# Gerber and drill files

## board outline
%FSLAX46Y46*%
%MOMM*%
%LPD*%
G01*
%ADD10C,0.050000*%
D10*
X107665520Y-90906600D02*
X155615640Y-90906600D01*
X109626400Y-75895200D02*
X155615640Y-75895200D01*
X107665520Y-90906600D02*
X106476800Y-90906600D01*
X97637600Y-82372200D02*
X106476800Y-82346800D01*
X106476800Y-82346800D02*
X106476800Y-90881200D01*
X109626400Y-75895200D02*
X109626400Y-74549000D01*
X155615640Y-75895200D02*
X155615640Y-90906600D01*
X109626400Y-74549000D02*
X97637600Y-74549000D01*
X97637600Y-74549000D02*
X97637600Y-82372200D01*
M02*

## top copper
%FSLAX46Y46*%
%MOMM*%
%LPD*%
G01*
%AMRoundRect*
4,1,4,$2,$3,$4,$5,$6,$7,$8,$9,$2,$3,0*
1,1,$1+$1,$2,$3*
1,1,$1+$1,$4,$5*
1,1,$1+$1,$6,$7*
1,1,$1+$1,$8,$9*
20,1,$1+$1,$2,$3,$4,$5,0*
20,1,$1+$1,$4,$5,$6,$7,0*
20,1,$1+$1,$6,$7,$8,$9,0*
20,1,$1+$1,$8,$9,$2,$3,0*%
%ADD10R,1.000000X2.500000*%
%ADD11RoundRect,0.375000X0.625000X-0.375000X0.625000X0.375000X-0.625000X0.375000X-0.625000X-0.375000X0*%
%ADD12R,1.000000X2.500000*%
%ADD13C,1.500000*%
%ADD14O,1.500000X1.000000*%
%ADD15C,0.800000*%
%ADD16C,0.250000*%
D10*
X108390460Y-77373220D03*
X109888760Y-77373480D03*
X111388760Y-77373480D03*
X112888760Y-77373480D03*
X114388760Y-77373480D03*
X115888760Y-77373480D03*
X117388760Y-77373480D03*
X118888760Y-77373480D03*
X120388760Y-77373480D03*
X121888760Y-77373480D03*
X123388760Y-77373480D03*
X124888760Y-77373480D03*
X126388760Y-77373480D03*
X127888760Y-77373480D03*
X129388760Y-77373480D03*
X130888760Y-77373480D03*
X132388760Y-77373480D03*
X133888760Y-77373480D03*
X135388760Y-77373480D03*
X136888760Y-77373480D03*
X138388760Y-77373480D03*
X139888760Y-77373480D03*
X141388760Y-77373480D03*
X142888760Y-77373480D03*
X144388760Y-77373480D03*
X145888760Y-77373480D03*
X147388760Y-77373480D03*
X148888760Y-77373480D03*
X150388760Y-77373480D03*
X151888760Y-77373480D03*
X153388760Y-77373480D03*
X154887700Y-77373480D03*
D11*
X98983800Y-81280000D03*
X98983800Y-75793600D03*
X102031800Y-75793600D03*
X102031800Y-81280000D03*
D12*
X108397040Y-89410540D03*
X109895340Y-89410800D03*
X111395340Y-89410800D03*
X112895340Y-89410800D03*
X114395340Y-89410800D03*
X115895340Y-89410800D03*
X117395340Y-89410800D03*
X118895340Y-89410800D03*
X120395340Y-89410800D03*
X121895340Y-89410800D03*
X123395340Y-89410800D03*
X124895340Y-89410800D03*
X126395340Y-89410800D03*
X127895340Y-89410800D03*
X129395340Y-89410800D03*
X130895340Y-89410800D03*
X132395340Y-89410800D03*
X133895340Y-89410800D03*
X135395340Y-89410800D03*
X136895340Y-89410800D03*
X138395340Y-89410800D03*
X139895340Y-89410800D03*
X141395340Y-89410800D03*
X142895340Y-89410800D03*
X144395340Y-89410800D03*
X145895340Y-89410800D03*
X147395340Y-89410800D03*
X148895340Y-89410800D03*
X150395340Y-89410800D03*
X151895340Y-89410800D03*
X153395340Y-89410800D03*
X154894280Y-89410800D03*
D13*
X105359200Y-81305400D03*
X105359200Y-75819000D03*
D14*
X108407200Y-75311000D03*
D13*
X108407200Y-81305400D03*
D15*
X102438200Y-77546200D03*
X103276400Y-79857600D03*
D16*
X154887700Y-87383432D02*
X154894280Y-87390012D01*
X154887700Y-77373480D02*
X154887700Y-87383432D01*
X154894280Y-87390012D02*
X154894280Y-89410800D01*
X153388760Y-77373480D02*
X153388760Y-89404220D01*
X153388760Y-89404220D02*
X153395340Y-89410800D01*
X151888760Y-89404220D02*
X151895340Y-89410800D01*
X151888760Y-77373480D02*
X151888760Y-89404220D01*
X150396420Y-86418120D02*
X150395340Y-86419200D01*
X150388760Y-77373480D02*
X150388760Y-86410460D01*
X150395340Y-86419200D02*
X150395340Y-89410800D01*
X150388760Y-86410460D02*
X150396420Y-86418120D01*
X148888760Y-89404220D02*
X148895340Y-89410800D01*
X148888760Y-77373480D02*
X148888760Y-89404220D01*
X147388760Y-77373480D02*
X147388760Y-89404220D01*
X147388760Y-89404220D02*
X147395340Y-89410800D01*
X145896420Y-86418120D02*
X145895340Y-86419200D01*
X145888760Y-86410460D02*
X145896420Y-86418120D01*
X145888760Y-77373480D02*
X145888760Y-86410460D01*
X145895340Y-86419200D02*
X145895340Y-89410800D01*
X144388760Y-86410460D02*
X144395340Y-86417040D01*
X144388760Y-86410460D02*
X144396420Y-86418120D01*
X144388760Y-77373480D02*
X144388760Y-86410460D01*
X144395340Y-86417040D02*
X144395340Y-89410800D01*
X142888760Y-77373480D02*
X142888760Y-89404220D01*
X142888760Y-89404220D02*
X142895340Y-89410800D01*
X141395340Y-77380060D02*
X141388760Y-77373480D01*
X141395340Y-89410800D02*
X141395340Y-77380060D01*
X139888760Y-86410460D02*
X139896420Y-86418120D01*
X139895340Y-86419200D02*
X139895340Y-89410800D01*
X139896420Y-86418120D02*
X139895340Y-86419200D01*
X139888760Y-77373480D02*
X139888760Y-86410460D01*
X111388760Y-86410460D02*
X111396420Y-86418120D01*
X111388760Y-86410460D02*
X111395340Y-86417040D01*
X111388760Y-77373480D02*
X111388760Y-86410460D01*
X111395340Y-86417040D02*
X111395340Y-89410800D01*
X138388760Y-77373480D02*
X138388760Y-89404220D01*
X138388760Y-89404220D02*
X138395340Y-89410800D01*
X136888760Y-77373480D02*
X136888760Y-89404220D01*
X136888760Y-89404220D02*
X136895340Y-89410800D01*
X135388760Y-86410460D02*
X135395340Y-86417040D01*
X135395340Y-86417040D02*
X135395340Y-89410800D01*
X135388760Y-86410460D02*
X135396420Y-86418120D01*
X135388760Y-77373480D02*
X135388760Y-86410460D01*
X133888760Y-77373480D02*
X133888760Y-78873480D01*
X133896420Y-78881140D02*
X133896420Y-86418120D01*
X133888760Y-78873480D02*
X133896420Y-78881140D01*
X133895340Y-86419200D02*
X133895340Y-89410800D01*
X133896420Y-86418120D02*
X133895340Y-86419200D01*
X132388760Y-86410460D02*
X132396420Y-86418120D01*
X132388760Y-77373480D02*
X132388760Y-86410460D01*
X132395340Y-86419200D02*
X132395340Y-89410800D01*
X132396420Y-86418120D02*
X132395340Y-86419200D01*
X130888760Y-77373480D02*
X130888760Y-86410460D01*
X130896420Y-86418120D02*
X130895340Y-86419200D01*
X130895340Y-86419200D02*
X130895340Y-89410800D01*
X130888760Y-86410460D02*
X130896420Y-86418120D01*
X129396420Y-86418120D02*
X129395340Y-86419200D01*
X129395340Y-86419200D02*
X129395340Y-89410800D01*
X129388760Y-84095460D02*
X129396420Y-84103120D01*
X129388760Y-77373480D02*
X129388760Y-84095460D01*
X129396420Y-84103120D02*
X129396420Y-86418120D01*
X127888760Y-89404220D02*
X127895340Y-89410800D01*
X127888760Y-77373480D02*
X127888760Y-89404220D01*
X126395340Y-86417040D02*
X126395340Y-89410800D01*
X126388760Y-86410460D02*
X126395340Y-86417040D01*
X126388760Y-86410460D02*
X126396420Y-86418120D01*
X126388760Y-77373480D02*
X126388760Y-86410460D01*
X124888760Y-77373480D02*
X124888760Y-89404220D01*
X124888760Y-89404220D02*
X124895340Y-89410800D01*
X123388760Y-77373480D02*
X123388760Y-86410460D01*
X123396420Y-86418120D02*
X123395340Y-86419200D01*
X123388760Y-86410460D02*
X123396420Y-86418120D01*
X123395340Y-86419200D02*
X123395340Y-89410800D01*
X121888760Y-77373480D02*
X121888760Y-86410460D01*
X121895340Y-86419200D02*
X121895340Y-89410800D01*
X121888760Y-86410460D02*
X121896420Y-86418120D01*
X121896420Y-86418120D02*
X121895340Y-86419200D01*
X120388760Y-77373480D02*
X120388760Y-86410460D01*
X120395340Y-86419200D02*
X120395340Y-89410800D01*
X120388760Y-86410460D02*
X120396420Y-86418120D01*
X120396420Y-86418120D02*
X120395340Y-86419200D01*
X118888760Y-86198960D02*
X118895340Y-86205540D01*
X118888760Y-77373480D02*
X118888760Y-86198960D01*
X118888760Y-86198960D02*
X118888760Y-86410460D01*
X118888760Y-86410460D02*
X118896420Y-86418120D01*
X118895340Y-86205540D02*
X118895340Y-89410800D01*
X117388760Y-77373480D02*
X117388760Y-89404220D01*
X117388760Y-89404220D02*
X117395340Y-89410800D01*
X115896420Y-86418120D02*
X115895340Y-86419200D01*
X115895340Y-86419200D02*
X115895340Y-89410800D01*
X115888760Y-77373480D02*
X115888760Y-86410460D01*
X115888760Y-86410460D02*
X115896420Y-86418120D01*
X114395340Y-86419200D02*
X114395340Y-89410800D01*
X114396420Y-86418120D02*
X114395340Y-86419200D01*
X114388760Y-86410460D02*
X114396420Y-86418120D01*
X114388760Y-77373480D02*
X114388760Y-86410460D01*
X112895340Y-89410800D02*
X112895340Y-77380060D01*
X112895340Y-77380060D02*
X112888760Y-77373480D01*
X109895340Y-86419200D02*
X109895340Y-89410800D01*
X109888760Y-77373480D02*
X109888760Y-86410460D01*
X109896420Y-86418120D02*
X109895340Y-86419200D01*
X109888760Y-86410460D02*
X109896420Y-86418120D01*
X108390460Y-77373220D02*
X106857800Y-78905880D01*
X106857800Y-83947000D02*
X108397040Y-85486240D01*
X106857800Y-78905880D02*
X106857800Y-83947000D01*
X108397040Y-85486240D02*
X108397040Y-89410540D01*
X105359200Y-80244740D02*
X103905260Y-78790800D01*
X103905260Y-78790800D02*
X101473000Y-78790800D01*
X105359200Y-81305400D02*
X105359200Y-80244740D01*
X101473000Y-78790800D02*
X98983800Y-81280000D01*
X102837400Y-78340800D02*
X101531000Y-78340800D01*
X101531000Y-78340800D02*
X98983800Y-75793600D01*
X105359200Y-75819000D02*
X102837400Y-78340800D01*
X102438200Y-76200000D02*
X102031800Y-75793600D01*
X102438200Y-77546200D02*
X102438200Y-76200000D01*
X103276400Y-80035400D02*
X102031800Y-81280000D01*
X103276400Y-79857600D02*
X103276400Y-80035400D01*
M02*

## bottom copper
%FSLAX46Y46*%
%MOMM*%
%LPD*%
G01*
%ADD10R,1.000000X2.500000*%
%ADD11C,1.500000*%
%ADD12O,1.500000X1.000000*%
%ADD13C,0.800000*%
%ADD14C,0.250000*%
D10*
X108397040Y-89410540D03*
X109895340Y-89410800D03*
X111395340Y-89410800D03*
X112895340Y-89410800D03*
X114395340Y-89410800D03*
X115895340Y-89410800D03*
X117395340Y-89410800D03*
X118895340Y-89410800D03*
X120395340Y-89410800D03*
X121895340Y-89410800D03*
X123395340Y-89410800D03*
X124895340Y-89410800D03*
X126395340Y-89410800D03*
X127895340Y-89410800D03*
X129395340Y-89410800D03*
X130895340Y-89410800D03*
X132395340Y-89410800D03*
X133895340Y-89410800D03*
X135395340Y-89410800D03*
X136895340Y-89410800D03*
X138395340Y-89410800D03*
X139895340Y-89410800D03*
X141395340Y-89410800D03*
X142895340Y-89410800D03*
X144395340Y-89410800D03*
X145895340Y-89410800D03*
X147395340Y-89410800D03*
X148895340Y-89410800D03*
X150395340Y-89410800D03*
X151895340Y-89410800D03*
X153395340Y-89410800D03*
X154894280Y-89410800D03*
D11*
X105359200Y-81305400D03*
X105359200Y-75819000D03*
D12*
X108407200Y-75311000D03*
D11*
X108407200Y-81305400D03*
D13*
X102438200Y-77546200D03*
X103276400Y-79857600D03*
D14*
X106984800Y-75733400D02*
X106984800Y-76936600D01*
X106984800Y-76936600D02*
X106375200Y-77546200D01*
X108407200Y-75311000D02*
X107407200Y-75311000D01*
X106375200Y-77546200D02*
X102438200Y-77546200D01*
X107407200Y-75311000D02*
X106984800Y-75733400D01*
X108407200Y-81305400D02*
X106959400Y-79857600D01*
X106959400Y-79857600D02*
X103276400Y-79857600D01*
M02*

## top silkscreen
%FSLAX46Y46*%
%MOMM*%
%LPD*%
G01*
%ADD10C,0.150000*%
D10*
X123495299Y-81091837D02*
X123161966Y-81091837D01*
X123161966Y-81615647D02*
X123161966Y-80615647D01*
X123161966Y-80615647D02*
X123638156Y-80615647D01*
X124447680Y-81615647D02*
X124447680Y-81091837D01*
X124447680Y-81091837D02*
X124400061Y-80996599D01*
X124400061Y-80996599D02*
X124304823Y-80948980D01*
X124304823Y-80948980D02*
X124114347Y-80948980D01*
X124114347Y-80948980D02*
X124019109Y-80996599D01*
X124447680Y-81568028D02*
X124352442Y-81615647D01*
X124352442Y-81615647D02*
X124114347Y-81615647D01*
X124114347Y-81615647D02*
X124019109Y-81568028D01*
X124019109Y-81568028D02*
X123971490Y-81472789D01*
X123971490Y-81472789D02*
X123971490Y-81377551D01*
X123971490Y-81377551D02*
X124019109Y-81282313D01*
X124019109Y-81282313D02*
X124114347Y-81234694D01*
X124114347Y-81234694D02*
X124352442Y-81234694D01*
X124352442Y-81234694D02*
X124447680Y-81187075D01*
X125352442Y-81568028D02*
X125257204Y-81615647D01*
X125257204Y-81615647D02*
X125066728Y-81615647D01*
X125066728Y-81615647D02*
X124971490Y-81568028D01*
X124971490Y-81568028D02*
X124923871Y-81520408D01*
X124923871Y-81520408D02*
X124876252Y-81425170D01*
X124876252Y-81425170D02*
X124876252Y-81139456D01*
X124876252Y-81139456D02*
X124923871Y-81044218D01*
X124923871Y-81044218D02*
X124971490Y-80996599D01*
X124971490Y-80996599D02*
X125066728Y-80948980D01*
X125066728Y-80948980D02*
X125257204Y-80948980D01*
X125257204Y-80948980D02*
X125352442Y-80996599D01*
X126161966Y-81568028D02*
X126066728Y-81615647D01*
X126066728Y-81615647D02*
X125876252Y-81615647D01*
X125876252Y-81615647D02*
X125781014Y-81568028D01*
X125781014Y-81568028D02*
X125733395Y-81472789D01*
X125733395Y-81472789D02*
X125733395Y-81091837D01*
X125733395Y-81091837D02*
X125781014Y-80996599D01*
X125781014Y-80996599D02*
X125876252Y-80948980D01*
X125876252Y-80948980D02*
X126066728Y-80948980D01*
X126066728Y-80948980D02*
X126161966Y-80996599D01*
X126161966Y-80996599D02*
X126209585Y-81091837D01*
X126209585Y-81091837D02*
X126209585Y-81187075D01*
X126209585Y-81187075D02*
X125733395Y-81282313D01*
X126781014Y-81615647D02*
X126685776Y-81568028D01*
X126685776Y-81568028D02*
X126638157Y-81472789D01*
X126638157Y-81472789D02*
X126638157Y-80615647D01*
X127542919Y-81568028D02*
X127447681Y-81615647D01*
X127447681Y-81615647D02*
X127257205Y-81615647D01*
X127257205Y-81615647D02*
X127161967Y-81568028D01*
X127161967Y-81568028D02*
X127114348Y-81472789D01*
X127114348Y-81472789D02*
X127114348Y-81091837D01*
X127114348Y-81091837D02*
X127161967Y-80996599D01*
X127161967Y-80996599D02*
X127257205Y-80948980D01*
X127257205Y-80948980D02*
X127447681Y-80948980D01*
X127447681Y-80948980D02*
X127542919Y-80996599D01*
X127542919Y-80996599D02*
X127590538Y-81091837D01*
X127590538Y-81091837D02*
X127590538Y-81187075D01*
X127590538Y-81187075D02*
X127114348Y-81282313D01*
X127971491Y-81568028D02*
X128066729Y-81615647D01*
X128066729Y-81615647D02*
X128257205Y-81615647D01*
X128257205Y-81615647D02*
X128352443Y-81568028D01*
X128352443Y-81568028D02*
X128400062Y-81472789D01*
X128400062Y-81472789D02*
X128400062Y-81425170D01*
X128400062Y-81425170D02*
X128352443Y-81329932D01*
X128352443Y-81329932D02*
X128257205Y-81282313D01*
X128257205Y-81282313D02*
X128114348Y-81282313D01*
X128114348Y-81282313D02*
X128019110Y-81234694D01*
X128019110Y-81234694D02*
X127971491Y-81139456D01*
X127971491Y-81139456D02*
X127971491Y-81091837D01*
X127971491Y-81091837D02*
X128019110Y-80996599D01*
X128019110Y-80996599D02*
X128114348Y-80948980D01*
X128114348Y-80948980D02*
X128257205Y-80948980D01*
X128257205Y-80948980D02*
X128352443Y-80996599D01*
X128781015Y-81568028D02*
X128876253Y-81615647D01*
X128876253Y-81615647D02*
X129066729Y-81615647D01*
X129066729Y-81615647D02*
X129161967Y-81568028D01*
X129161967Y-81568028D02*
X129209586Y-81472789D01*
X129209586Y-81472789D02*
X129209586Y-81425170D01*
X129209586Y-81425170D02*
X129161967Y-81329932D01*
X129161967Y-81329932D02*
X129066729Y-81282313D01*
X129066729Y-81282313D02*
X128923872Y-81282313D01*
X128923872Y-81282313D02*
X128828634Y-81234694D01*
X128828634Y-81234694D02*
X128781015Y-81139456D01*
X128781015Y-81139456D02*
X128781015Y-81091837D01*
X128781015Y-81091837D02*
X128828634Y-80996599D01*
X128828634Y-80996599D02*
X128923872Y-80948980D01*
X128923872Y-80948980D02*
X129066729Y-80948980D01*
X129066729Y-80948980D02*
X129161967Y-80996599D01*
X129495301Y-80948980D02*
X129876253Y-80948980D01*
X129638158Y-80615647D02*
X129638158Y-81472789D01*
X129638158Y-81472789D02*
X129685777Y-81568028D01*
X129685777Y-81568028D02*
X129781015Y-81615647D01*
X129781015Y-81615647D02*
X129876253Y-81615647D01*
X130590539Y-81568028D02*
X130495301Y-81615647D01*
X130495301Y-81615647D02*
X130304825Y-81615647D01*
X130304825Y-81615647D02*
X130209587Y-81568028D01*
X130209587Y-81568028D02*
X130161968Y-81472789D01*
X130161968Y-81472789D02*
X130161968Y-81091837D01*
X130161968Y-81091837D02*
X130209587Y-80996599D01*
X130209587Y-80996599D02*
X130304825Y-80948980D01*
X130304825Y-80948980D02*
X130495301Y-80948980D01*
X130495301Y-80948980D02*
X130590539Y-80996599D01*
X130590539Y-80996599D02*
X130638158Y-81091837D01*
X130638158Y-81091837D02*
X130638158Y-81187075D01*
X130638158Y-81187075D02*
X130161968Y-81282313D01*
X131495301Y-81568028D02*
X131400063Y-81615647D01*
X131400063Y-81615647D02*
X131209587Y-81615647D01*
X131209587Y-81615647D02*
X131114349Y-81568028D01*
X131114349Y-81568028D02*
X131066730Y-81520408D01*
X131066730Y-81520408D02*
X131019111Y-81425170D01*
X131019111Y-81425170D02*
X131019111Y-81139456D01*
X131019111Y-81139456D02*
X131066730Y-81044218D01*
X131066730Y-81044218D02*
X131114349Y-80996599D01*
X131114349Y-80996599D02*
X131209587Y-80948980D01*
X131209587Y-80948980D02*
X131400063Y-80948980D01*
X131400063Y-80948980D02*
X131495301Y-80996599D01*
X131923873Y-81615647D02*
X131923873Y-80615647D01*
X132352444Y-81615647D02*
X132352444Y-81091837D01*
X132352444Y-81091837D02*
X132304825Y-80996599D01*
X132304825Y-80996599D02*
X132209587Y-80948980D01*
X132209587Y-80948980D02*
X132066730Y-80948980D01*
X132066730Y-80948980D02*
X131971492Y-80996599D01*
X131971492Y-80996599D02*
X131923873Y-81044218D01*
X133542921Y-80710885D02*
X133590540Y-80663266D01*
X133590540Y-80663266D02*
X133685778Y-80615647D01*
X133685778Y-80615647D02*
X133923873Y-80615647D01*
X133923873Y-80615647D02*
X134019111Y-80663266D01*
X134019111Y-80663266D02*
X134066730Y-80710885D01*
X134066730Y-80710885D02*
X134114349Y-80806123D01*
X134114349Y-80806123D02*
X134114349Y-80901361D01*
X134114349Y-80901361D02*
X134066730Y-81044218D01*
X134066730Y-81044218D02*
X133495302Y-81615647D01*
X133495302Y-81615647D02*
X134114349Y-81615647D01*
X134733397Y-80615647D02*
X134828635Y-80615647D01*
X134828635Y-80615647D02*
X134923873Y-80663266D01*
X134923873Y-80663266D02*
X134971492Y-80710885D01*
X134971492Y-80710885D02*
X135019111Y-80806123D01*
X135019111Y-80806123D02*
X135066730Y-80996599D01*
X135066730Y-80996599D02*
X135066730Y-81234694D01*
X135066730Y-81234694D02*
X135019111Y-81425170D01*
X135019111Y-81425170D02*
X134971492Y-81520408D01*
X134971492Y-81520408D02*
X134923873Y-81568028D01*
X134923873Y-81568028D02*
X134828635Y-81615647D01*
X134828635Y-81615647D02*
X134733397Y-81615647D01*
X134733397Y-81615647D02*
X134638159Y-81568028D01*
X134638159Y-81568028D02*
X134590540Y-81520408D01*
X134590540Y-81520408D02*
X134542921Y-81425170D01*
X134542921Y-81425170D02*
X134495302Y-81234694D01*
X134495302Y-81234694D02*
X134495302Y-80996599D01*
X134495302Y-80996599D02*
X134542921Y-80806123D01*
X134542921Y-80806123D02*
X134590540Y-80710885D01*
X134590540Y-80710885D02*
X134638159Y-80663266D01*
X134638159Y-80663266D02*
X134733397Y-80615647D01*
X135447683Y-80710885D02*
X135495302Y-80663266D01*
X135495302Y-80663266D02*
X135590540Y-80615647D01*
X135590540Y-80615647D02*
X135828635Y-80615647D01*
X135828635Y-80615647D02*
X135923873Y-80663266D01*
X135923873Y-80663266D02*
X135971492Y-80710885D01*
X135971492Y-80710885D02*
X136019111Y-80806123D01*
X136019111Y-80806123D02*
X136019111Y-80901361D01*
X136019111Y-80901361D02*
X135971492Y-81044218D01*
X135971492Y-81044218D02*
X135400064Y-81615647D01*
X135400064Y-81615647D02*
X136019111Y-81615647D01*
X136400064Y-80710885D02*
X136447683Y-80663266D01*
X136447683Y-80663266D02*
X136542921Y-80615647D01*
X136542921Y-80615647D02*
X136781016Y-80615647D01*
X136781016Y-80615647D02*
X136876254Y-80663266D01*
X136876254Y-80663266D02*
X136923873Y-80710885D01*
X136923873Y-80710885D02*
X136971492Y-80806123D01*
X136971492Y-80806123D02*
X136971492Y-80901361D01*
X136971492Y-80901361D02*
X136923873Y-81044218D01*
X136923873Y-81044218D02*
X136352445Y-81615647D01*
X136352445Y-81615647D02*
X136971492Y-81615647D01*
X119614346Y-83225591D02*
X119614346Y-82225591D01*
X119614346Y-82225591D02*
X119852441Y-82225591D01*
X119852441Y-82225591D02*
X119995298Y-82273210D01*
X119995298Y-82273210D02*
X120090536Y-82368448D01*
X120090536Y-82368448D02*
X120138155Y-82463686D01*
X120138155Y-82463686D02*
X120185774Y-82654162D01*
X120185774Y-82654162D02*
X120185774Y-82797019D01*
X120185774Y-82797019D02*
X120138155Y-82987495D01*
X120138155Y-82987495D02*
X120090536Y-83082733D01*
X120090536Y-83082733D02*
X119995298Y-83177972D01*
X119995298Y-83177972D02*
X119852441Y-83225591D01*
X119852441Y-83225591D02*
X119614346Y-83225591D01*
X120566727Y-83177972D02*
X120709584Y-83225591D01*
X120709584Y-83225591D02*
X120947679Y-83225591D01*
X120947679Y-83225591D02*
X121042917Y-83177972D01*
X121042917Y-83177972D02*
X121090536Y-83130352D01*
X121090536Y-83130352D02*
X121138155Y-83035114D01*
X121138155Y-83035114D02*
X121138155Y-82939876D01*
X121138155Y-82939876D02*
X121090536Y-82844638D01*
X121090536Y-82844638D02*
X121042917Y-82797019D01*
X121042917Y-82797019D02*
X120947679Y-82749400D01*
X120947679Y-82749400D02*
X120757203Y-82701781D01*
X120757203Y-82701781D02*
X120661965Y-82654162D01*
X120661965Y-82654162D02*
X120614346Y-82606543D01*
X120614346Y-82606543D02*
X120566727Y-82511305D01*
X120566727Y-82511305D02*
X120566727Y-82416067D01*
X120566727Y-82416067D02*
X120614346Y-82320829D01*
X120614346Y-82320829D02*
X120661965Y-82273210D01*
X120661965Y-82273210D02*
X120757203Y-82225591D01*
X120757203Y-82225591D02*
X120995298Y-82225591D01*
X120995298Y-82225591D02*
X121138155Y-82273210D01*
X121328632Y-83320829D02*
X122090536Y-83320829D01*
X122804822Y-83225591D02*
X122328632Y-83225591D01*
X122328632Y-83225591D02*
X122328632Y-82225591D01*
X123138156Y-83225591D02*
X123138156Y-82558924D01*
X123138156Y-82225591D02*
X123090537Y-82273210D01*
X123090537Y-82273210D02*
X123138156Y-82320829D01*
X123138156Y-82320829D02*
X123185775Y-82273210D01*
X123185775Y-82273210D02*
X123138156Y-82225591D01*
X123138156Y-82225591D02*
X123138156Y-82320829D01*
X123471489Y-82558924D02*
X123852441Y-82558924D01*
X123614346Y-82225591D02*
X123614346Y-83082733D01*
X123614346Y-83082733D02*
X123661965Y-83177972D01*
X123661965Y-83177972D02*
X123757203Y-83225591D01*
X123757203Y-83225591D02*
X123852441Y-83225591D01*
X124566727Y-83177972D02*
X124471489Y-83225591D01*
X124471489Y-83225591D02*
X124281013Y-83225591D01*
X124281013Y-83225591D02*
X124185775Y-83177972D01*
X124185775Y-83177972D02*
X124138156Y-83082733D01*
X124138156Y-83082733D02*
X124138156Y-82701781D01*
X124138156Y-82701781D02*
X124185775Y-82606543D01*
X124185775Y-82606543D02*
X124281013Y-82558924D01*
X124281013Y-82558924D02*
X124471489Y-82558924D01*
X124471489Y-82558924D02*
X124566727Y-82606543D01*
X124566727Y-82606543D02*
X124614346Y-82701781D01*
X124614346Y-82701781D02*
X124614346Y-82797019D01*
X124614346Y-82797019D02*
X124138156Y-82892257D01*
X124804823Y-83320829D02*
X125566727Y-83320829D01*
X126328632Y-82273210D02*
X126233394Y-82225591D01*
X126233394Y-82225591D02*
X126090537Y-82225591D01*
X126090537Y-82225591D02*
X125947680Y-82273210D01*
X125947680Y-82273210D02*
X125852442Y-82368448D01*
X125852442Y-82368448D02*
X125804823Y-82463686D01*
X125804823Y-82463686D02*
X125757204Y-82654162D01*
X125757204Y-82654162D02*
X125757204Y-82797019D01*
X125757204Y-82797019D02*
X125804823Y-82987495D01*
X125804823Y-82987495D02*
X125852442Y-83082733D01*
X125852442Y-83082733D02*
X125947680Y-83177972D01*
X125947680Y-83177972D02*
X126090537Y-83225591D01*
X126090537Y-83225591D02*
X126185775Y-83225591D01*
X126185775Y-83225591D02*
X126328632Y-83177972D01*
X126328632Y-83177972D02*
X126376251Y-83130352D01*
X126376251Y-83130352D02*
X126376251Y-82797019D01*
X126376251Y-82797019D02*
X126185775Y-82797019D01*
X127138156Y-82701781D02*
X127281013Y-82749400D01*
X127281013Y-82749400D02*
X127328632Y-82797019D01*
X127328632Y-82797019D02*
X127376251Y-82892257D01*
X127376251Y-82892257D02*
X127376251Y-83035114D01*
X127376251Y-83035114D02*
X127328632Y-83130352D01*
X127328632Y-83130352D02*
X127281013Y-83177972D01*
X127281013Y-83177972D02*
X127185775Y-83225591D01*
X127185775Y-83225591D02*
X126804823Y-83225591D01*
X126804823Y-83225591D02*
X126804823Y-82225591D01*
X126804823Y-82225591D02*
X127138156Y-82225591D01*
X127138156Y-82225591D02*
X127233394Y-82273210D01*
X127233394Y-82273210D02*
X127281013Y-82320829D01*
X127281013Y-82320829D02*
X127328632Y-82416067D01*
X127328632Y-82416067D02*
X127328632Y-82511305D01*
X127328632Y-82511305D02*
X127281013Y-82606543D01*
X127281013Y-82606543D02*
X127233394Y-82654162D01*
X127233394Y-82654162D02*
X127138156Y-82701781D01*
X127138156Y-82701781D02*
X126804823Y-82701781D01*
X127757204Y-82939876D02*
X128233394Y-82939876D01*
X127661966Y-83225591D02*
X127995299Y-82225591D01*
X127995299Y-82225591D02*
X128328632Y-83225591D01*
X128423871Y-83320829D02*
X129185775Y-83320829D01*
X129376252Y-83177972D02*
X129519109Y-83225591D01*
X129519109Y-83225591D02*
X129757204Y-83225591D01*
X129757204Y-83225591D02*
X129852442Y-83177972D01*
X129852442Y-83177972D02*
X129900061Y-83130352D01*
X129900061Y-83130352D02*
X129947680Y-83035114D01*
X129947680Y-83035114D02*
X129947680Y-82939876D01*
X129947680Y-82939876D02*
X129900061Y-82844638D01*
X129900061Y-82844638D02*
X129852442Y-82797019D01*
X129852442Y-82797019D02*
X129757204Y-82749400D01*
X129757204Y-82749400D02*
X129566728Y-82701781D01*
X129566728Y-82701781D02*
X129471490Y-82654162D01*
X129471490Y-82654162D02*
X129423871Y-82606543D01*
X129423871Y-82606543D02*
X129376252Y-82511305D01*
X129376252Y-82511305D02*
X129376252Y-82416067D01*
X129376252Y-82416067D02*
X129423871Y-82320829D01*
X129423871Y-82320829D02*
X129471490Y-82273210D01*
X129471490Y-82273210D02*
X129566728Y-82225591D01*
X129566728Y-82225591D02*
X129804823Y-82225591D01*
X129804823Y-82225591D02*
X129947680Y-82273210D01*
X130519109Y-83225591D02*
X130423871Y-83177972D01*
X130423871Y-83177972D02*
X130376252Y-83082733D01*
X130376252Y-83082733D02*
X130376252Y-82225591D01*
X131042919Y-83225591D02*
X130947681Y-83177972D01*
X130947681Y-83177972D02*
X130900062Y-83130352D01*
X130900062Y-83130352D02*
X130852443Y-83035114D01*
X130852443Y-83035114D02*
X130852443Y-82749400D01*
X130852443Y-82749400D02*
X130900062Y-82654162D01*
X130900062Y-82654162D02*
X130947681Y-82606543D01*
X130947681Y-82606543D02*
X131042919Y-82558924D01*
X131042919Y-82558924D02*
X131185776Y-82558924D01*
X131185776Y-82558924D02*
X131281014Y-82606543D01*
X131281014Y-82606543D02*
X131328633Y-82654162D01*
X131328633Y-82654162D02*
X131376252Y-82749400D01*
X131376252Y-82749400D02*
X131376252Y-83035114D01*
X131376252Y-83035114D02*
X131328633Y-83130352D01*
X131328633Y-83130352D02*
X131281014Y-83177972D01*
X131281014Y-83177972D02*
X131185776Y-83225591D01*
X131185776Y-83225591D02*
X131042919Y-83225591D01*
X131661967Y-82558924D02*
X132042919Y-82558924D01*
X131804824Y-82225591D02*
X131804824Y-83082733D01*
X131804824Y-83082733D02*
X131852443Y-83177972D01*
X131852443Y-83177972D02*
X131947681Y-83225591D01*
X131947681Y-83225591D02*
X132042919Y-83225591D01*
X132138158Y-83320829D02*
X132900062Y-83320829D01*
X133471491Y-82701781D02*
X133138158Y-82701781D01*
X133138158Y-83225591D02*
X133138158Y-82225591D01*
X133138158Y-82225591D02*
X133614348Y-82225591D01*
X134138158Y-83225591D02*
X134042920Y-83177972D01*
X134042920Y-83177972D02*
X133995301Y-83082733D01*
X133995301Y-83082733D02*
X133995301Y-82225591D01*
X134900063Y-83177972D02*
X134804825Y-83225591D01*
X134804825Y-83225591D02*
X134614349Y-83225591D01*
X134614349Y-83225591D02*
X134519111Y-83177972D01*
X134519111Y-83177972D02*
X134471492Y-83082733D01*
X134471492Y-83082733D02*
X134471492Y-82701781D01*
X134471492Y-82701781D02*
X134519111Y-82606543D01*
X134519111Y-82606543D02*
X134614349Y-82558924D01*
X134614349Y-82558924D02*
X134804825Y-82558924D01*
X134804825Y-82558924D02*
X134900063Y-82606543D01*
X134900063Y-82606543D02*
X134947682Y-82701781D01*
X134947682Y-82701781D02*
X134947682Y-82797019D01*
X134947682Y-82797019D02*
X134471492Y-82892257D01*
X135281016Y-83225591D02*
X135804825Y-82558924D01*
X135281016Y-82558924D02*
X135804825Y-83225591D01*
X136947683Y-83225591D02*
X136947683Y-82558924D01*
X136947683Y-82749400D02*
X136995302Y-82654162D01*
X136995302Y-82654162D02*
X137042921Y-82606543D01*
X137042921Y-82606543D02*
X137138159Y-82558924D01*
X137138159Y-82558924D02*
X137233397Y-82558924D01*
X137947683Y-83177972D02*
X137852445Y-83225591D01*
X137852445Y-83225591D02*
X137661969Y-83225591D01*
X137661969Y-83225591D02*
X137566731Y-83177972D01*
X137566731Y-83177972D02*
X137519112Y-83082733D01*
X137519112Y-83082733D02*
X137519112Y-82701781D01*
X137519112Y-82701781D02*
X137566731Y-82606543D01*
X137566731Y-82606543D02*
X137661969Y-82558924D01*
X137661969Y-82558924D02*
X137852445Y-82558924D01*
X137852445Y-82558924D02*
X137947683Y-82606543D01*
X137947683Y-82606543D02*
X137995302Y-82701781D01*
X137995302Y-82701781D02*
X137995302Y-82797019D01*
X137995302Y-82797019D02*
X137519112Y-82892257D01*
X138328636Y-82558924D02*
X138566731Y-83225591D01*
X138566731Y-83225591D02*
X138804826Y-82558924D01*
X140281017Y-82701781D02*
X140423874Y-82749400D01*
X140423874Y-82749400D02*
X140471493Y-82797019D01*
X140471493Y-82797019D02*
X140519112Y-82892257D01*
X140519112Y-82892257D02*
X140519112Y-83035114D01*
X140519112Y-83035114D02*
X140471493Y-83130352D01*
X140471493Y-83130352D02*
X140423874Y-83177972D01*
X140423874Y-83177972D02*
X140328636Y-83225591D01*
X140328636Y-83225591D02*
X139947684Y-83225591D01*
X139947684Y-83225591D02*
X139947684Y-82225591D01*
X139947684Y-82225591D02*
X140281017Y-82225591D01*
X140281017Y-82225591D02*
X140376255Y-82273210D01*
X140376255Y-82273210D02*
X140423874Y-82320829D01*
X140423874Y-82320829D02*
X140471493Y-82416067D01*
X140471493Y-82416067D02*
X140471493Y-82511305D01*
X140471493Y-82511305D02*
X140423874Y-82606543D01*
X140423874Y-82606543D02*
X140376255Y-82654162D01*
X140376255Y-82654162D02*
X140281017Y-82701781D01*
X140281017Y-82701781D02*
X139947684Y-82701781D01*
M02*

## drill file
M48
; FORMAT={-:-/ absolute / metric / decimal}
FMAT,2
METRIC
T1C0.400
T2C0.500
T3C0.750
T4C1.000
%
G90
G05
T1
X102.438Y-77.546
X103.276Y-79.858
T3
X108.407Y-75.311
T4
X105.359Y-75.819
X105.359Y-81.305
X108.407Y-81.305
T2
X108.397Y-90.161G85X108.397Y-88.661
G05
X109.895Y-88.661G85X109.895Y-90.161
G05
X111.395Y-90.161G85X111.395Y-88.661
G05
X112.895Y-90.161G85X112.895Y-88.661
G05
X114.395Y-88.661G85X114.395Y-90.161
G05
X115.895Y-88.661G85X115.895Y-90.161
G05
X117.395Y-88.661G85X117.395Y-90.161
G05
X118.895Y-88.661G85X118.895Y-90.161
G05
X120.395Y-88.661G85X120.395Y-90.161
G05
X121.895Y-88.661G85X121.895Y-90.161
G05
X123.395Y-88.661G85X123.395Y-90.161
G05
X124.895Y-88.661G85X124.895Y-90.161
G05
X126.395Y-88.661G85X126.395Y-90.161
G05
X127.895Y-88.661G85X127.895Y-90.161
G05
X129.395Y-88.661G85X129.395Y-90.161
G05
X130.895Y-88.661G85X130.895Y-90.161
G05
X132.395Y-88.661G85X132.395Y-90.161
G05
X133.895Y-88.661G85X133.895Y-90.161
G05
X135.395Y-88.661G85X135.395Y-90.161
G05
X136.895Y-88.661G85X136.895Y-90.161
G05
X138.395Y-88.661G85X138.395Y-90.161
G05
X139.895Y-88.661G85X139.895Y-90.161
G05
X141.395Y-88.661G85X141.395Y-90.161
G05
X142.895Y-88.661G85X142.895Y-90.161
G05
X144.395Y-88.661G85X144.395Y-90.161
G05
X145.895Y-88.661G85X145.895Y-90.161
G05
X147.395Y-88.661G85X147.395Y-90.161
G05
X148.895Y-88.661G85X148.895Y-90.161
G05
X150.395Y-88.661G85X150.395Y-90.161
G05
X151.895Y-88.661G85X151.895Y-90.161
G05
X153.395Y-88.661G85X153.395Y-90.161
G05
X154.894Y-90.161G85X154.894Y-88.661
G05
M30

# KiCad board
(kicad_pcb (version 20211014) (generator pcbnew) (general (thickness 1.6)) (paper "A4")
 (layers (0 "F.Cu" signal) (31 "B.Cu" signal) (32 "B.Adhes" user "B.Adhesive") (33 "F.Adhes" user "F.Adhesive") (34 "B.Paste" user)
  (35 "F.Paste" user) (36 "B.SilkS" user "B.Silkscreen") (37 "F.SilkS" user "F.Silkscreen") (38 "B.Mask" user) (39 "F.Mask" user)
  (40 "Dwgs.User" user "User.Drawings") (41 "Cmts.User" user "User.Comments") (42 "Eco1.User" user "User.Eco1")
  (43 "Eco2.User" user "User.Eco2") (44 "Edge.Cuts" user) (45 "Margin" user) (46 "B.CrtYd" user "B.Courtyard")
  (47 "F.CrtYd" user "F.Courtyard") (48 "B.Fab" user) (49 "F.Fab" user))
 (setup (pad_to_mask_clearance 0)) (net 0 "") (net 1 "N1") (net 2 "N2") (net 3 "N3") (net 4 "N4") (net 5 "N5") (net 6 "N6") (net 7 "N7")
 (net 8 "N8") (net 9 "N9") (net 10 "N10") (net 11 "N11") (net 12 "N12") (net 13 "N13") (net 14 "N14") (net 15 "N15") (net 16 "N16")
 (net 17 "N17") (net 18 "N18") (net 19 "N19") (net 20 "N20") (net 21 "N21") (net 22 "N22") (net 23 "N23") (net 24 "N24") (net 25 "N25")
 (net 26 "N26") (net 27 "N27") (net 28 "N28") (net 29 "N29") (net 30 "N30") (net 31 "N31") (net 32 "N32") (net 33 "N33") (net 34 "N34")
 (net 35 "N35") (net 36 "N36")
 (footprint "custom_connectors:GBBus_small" (layer "F.Cu") (at 130.11762 77.37068)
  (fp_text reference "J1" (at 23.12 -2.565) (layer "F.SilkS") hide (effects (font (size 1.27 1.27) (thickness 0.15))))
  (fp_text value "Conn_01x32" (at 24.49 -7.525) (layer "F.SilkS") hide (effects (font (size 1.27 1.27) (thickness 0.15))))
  (pad "1" smd rect locked (at -21.72716 0.00254 180) (size 1 2.5) (layers "F.Cu" "F.Paste" "F.Mask") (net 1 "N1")
   (solder_mask_margin 0.0508))
  (pad "2" smd rect locked (at -20.22886 0.0028) (size 1 2.5) (layers "F.Cu" "F.Paste" "F.Mask") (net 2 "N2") (solder_mask_margin 0.0508))
  (pad "3" smd rect locked (at -18.72886 0.0028 180) (size 1 2.5) (layers "F.Cu" "F.Paste" "F.Mask") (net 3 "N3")
   (solder_mask_margin 0.0508))
  (pad "4" smd rect locked (at -17.22886 0.0028 180) (size 1 2.5) (layers "F.Cu" "F.Paste" "F.Mask") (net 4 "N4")
   (solder_mask_margin 0.0508))
  (pad "5" smd rect locked (at -15.72886 0.0028) (size 1 2.5) (layers "F.Cu" "F.Paste" "F.Mask") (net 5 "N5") (solder_mask_margin 0.0508))
  (pad "6" smd rect locked (at -14.22886 0.0028) (size 1 2.5) (layers "F.Cu" "F.Paste" "F.Mask") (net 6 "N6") (solder_mask_margin 0.0508))
  (pad "7" smd rect locked (at -12.72886 0.0028) (size 1 2.5) (layers "F.Cu" "F.Paste" "F.Mask") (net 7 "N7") (solder_mask_margin 0.0508))
  (pad "8" smd rect locked (at -11.22886 0.0028) (size 1 2.5) (layers "F.Cu" "F.Paste" "F.Mask") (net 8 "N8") (solder_mask_margin 0.0508))
  (pad "9" smd rect locked (at -9.72886 0.0028) (size 1 2.5) (layers "F.Cu" "F.Paste" "F.Mask") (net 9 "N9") (solder_mask_margin 0.0508))
  (pad "10" smd rect locked (at -8.22886 0.0028) (size 1 2.5) (layers "F.Cu" "F.Paste" "F.Mask") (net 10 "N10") (solder_mask_margin 0.0508))
  (pad "11" smd rect locked (at -6.72886 0.0028) (size 1 2.5) (layers "F.Cu" "F.Paste" "F.Mask") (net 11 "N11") (solder_mask_margin 0.0508))
  (pad "12" smd rect locked (at -5.22886 0.0028) (size 1 2.5) (layers "F.Cu" "F.Paste" "F.Mask") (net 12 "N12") (solder_mask_margin 0.0508))
  (pad "13" smd rect locked (at -3.72886 0.0028) (size 1 2.5) (layers "F.Cu" "F.Paste" "F.Mask") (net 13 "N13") (solder_mask_margin 0.0508))
  (pad "14" smd rect locked (at -2.22886 0.0028) (size 1 2.5) (layers "F.Cu" "F.Paste" "F.Mask") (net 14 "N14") (solder_mask_margin 0.0508))
  (pad "15" smd rect locked (at -0.72886 0.0028) (size 1 2.5) (layers "F.Cu" "F.Paste" "F.Mask") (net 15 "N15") (solder_mask_margin 0.0508))
  (pad "16" smd rect locked (at 0.77114 0.0028) (size 1 2.5) (layers "F.Cu" "F.Paste" "F.Mask") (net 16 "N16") (solder_mask_margin 0.0508))
  (pad "17" smd rect locked (at 2.27114 0.0028) (size 1 2.5) (layers "F.Cu" "F.Paste" "F.Mask") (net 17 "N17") (solder_mask_margin 0.0508))
  (pad "18" smd rect locked (at 3.77114 0.0028) (size 1 2.5) (layers "F.Cu" "F.Paste" "F.Mask") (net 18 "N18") (solder_mask_margin 0.0508))
  (pad "19" smd rect locked (at 5.27114 0.0028) (size 1 2.5) (layers "F.Cu" "F.Paste" "F.Mask") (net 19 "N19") (solder_mask_margin 0.0508))
  (pad "20" smd rect locked (at 6.77114 0.0028) (size 1 2.5) (layers "F.Cu" "F.Paste" "F.Mask") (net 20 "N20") (solder_mask_margin 0.0508))
  (pad "21" smd rect locked (at 8.27114 0.0028) (size 1 2.5) (layers "F.Cu" "F.Paste" "F.Mask") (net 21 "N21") (solder_mask_margin 0.0508))
  (pad "22" smd rect locked (at 9.77114 0.0028) (size 1 2.5) (layers "F.Cu" "F.Paste" "F.Mask") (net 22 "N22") (solder_mask_margin 0.0508))
  (pad "23" smd rect locked (at 11.27114 0.0028) (size 1 2.5) (layers "F.Cu" "F.Paste" "F.Mask") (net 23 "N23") (solder_mask_margin 0.0508))
  (pad "24" smd rect locked (at 12.77114 0.0028) (size 1 2.5) (layers "F.Cu" "F.Paste" "F.Mask") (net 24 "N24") (solder_mask_margin 0.0508))
  (pad "25" smd rect locked (at 14.27114 0.0028) (size 1 2.5) (layers "F.Cu" "F.Paste" "F.Mask") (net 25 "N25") (solder_mask_margin 0.0508))
  (pad "26" smd rect locked (at 15.77114 0.0028) (size 1 2.5) (layers "F.Cu" "F.Paste" "F.Mask") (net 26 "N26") (solder_mask_margin 0.0508))
  (pad "27" smd rect locked (at 17.27114 0.0028) (size 1 2.5) (layers "F.Cu" "F.Paste" "F.Mask") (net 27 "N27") (solder_mask_margin 0.0508))
  (pad "28" smd rect locked (at 18.77114 0.0028) (size 1 2.5) (layers "F.Cu" "F.Paste" "F.Mask") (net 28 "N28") (solder_mask_margin 0.0508))
  (pad "29" smd rect locked (at 20.27114 0.0028) (size 1 2.5) (layers "F.Cu" "F.Paste" "F.Mask") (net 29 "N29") (solder_mask_margin 0.0508))
  (pad "30" smd rect locked (at 21.77114 0.0028) (size 1 2.5) (layers "F.Cu" "F.Paste" "F.Mask") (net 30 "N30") (solder_mask_margin 0.0508))
  (pad "31" smd rect locked (at 23.27114 0.0028) (size 1 2.5) (layers "F.Cu" "F.Paste" "F.Mask") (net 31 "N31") (solder_mask_margin 0.0508))
  (pad "32" smd rect locked (at 24.77008 0.0028 180) (size 1 2.5) (layers "F.Cu" "F.Paste" "F.Mask") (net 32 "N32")
   (solder_mask_margin 0.0508)))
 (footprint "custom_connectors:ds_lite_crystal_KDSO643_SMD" (layer "F.Cu") (at 100.5078 78.5368 90)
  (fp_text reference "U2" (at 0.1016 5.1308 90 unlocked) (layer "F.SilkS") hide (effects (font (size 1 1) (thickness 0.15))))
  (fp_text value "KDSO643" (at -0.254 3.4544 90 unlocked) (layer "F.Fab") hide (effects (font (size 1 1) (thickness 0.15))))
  (pad "1" smd roundrect (at -2.7432 -1.524 90) (size 1.5 2) (layers "F.Cu" "F.Paste" "F.Mask") (roundrect_rratio 0.25) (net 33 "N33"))
  (pad "2" smd roundrect (at 2.7432 -1.524 90) (size 1.5 2) (layers "F.Cu" "F.Paste" "F.Mask") (roundrect_rratio 0.25) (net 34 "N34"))
  (pad "3" smd roundrect (at 2.7432 1.524 90) (size 1.5 2) (layers "F.Cu" "F.Paste" "F.Mask") (roundrect_rratio 0.25) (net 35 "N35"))
  (pad "4" smd roundrect (at -2.7432 1.524 90) (size 1.5 2) (layers "F.Cu" "F.Paste" "F.Mask") (roundrect_rratio 0.25) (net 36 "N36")))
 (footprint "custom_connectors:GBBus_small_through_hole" (layer "F.Cu") (at 130.1242 89.408)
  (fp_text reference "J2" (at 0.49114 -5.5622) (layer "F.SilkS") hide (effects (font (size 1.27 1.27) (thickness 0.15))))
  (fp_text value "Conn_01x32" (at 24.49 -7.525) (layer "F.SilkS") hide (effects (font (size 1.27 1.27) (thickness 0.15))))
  (pad "1" thru_hole rect (at -21.72716 0.00254 180) (size 1 2.5) (drill oval 0.5 2) (layers *.Cu *.Mask) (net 1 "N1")
   (solder_mask_margin 0.0508))
  (pad "2" thru_hole rect (at -20.22886 0.0028) (size 1 2.5) (drill oval 0.5 2) (layers *.Cu *.Mask) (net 2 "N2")
   (solder_mask_margin 0.0508))
  (pad "3" thru_hole rect (at -18.72886 0.0028 180) (size 1 2.5) (drill oval 0.5 2) (layers *.Cu *.Mask) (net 3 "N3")
   (solder_mask_margin 0.0508))
  (pad "4" thru_hole rect (at -17.22886 0.0028 180) (size 1 2.5) (drill oval 0.5 2) (layers *.Cu *.Mask) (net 4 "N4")
   (solder_mask_margin 0.0508))
  (pad "5" thru_hole rect (at -15.72886 0.0028) (size 1 2.5) (drill oval 0.5 2) (layers *.Cu *.Mask) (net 5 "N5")
   (solder_mask_margin 0.0508))
  (pad "6" thru_hole rect (at -14.22886 0.0028) (size 1 2.5) (drill oval 0.5 2) (layers *.Cu *.Mask) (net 6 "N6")
   (solder_mask_margin 0.0508))
  (pad "7" thru_hole rect (at -12.72886 0.0028) (size 1 2.5) (drill oval 0.5 2) (layers *.Cu *.Mask) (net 7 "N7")
   (solder_mask_margin 0.0508))
  (pad "8" thru_hole rect (at -11.22886 0.0028) (size 1 2.5) (drill oval 0.5 2) (layers *.Cu *.Mask) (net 8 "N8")
   (solder_mask_margin 0.0508))
  (pad "9" thru_hole rect (at -9.72886 0.0028) (size 1 2.5) (drill oval 0.5 2) (layers *.Cu *.Mask) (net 9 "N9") (solder_mask_margin 0.0508))
  (pad "10" thru_hole rect (at -8.22886 0.0028) (size 1 2.5) (drill oval 0.5 2) (layers *.Cu *.Mask) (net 10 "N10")
   (solder_mask_margin 0.0508))
  (pad "11" thru_hole rect (at -6.72886 0.0028) (size 1 2.5) (drill oval 0.5 2) (layers *.Cu *.Mask) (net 11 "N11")
   (solder_mask_margin 0.0508))
  (pad "12" thru_hole rect (at -5.22886 0.0028) (size 1 2.5) (drill oval 0.5 2) (layers *.Cu *.Mask) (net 12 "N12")
   (solder_mask_margin 0.0508))
  (pad "13" thru_hole rect (at -3.72886 0.0028) (size 1 2.5) (drill oval 0.5 2) (layers *.Cu *.Mask) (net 13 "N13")
   (solder_mask_margin 0.0508))
  (pad "14" thru_hole rect (at -2.22886 0.0028) (size 1 2.5) (drill oval 0.5 2) (layers *.Cu *.Mask) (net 14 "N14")
   (solder_mask_margin 0.0508))
  (pad "15" thru_hole rect (at -0.72886 0.0028) (size 1 2.5) (drill oval 0.5 2) (layers *.Cu *.Mask) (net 15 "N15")
   (solder_mask_margin 0.0508))
  (pad "16" thru_hole rect (at 0.77114 0.0028) (size 1 2.5) (drill oval 0.5 2) (layers *.Cu *.Mask) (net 16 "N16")
   (solder_mask_margin 0.0508))
  (pad "17" thru_hole rect (at 2.27114 0.0028) (size 1 2.5) (drill oval 0.5 2) (layers *.Cu *.Mask) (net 17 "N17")
   (solder_mask_margin 0.0508))
  (pad "18" thru_hole rect (at 3.77114 0.0028) (size 1 2.5) (drill oval 0.5 2) (layers *.Cu *.Mask) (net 18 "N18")
   (solder_mask_margin 0.0508))
  (pad "19" thru_hole rect (at 5.27114 0.0028) (size 1 2.5) (drill oval 0.5 2) (layers *.Cu *.Mask) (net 19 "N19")
   (solder_mask_margin 0.0508))
  (pad "20" thru_hole rect (at 6.77114 0.0028) (size 1 2.5) (drill oval 0.5 2) (layers *.Cu *.Mask) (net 20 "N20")
   (solder_mask_margin 0.0508))
  (pad "21" thru_hole rect (at 8.27114 0.0028) (size 1 2.5) (drill oval 0.5 2) (layers *.Cu *.Mask) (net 21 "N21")
   (solder_mask_margin 0.0508))
  (pad "22" thru_hole rect (at 9.77114 0.0028) (size 1 2.5) (drill oval 0.5 2) (layers *.Cu *.Mask) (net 22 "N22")
   (solder_mask_margin 0.0508))
  (pad "23" thru_hole rect (at 11.27114 0.0028) (size 1 2.5) (drill oval 0.5 2) (layers *.Cu *.Mask) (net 23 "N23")
   (solder_mask_margin 0.0508))
  (pad "24" thru_hole rect (at 12.77114 0.0028) (size 1 2.5) (drill oval 0.5 2) (layers *.Cu *.Mask) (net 24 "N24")
   (solder_mask_margin 0.0508))
  (pad "25" thru_hole rect (at 14.27114 0.0028) (size 1 2.5) (drill oval 0.5 2) (layers *.Cu *.Mask) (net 25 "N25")
   (solder_mask_margin 0.0508))
  (pad "26" thru_hole rect (at 15.77114 0.0028) (size 1 2.5) (drill oval 0.5 2) (layers *.Cu *.Mask) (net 26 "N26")
   (solder_mask_margin 0.0508))
  (pad "27" thru_hole rect (at 17.27114 0.0028) (size 1 2.5) (drill oval 0.5 2) (layers *.Cu *.Mask) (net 27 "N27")
   (solder_mask_margin 0.0508))
  (pad "28" thru_hole rect (at 18.77114 0.0028) (size 1 2.5) (drill oval 0.5 2) (layers *.Cu *.Mask) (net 28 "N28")
   (solder_mask_margin 0.0508))
  (pad "29" thru_hole rect (at 20.27114 0.0028) (size 1 2.5) (drill oval 0.5 2) (layers *.Cu *.Mask) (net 29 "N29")
   (solder_mask_margin 0.0508))
  (pad "30" thru_hole rect (at 21.77114 0.0028) (size 1 2.5) (drill oval 0.5 2) (layers *.Cu *.Mask) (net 30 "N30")
   (solder_mask_margin 0.0508))
  (pad "31" thru_hole rect (at 23.27114 0.0028) (size 1 2.5) (drill oval 0.5 2) (layers *.Cu *.Mask) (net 31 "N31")
   (solder_mask_margin 0.0508))
  (pad "32" thru_hole rect (at 24.77008 0.0028 180) (size 1 2.5) (drill oval 0.5 2) (layers *.Cu *.Mask) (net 32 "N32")
   (solder_mask_margin 0.0508)))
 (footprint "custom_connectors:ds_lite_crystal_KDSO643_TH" (layer "F.Cu") (at 106.8832 78.5622 90)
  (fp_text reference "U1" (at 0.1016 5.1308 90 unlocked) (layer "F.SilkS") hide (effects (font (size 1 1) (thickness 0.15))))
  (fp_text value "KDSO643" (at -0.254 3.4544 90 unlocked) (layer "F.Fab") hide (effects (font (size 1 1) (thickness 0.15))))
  (pad "1" thru_hole circle (at -2.7432 -1.524 90) (size 1.5 1.5) (drill 1) (layers *.Cu *.Mask) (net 33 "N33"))
  (pad "2" thru_hole circle (at 2.7432 -1.524 90) (size 1.5 1.5) (drill 1) (layers *.Cu *.Mask) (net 34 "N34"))
  (pad "3" thru_hole oval (at 3.2512 1.524 90) (size 1 1.5) (drill 0.75) (layers *.Cu *.Mask) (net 35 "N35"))
  (pad "4" thru_hole circle (at -2.7432 1.524 90) (size 1.5 1.5) (drill 1) (layers *.Cu *.Mask) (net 36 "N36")))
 (gr_line (start 107.66552 90.9066) (end 155.61564 90.9066) (layer "Edge.Cuts") (width 0.05))
 (gr_line (start 109.6264 75.8952) (end 155.61564 75.8952) (layer "Edge.Cuts") (width 0.05))
 (gr_line (start 107.66552 90.9066) (end 106.4768 90.9066) (layer "Edge.Cuts") (width 0.05))
 (gr_line (start 97.6376 82.3722) (end 106.4768 82.3468) (layer "Edge.Cuts") (width 0.05))
 (gr_line (start 106.4768 82.3468) (end 106.4768 90.8812) (layer "Edge.Cuts") (width 0.05))
 (gr_line (start 109.6264 75.8952) (end 109.6264 74.549) (layer "Edge.Cuts") (width 0.05))
 (gr_line (start 155.61564 75.8952) (end 155.61564 90.9066) (layer "Edge.Cuts") (width 0.05))
 (gr_line (start 109.6264 74.549) (end 97.6376 74.549) (layer "Edge.Cuts") (width 0.05))
 (gr_line (start 97.6376 74.549) (end 97.6376 82.3722) (layer "Edge.Cuts") (width 0.05))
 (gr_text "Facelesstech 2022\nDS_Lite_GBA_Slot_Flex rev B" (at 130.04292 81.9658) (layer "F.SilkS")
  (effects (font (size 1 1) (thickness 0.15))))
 (segment (start 154.8877 87.383432) (end 154.89428 87.390012) (width 0.25) (layer "F.Cu") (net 32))
 (segment (start 154.8877 77.37348) (end 154.8877 87.383432) (width 0.25) (layer "F.Cu") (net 32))
 (segment (start 154.89428 87.390012) (end 154.89428 89.4108) (width 0.25) (layer "F.Cu") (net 32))
 (segment (start 153.38876 77.37348) (end 153.38876 89.40422) (width 0.25) (layer "F.Cu") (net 31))
 (segment (start 153.38876 89.40422) (end 153.39534 89.4108) (width 0.25) (layer "F.Cu") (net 31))
 (segment (start 151.88876 89.40422) (end 151.89534 89.4108) (width 0.25) (layer "F.Cu") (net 30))
 (segment (start 151.88876 77.37348) (end 151.88876 89.40422) (width 0.25) (layer "F.Cu") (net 30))
 (segment (start 150.39642 86.41812) (end 150.39534 86.4192) (width 0.25) (layer "F.Cu") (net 29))
 (segment (start 150.38876 77.37348) (end 150.38876 86.41046) (width 0.25) (layer "F.Cu") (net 29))
 (segment (start 150.39534 86.4192) (end 150.39534 89.4108) (width 0.25) (layer "F.Cu") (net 29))
 (segment (start 150.38876 86.41046) (end 150.39642 86.41812) (width 0.25) (layer "F.Cu") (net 29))
 (segment (start 148.88876 89.40422) (end 148.89534 89.4108) (width 0.25) (layer "F.Cu") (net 28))
 (segment (start 148.88876 77.37348) (end 148.88876 89.40422) (width 0.25) (layer "F.Cu") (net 28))
 (segment (start 147.38876 77.37348) (end 147.38876 89.40422) (width 0.25) (layer "F.Cu") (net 27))
 (segment (start 147.38876 89.40422) (end 147.39534 89.4108) (width 0.25) (layer "F.Cu") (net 27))
 (segment (start 145.89642 86.41812) (end 145.89534 86.4192) (width 0.25) (layer "F.Cu") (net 26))
 (segment (start 145.88876 86.41046) (end 145.89642 86.41812) (width 0.25) (layer "F.Cu") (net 26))
 (segment (start 145.88876 77.37348) (end 145.88876 86.41046) (width 0.25) (layer "F.Cu") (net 26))
 (segment (start 145.89534 86.4192) (end 145.89534 89.4108) (width 0.25) (layer "F.Cu") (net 26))
 (segment (start 144.38876 86.41046) (end 144.39534 86.41704) (width 0.25) (layer "F.Cu") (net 25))
 (segment (start 144.38876 86.41046) (end 144.39642 86.41812) (width 0.25) (layer "F.Cu") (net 25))
 (segment (start 144.38876 77.37348) (end 144.38876 86.41046) (width 0.25) (layer "F.Cu") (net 25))
 (segment (start 144.39534 86.41704) (end 144.39534 89.4108) (width 0.25) (layer "F.Cu") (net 25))
 (segment (start 142.88876 77.37348) (end 142.88876 89.40422) (width 0.25) (layer "F.Cu") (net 24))
 (segment (start 142.88876 89.40422) (end 142.89534 89.4108) (width 0.25) (layer "F.Cu") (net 24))
 (segment (start 141.39534 77.38006) (end 141.38876 77.37348) (width 0.25) (layer "F.Cu") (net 23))
 (segment (start 141.39534 89.4108) (end 141.39534 77.38006) (width 0.25) (layer "F.Cu") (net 23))
 (segment (start 139.88876 86.41046) (end 139.89642 86.41812) (width 0.25) (layer "F.Cu") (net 22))
 (segment (start 139.89534 86.4192) (end 139.89534 89.4108) (width 0.25) (layer "F.Cu") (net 22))
 (segment (start 139.89642 86.41812) (end 139.89534 86.4192) (width 0.25) (layer "F.Cu") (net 22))
 (segment (start 139.88876 77.37348) (end 139.88876 86.41046) (width 0.25) (layer "F.Cu") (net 22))
 (segment (start 111.38876 86.41046) (end 111.39642 86.41812) (width 0.25) (layer "F.Cu") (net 3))
 (segment (start 111.38876 86.41046) (end 111.39534 86.41704) (width 0.25) (layer "F.Cu") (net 3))
 (segment (start 111.38876 77.37348) (end 111.38876 86.41046) (width 0.25) (layer "F.Cu") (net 3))
 (segment (start 111.39534 86.41704) (end 111.39534 89.4108) (width 0.25) (layer "F.Cu") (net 3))
 (segment (start 138.38876 77.37348) (end 138.38876 89.40422) (width 0.25) (layer "F.Cu") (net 21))
 (segment (start 138.38876 89.40422) (end 138.39534 89.4108) (width 0.25) (layer "F.Cu") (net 21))
 (segment (start 136.88876 77.37348) (end 136.88876 89.40422) (width 0.25) (layer "F.Cu") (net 20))
 (segment (start 136.88876 89.40422) (end 136.89534 89.4108) (width 0.25) (layer "F.Cu") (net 20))
 (segment (start 135.38876 86.41046) (end 135.39534 86.41704) (width 0.25) (layer "F.Cu") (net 19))
 (segment (start 135.39534 86.41704) (end 135.39534 89.4108) (width 0.25) (layer "F.Cu") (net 19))
 (segment (start 135.38876 86.41046) (end 135.39642 86.41812) (width 0.25) (layer "F.Cu") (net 19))
 (segment (start 135.38876 77.37348) (end 135.38876 86.41046) (width 0.25) (layer "F.Cu") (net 19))
 (segment (start 133.88876 77.37348) (end 133.88876 78.87348) (width 0.25) (layer "F.Cu") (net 18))
 (segment (start 133.89642 78.88114) (end 133.89642 86.41812) (width 0.25) (layer "F.Cu") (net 18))
 (segment (start 133.88876 78.87348) (end 133.89642 78.88114) (width 0.25) (layer "F.Cu") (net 18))
 (segment (start 133.89534 86.4192) (end 133.89534 89.4108) (width 0.25) (layer "F.Cu") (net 18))
 (segment (start 133.89642 86.41812) (end 133.89534 86.4192) (width 0.25) (layer "F.Cu") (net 18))
 (segment (start 132.38876 86.41046) (end 132.39642 86.41812) (width 0.25) (layer "F.Cu") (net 17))
 (segment (start 132.38876 77.37348) (end 132.38876 86.41046) (width 0.25) (layer "F.Cu") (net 17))
 (segment (start 132.39534 86.4192) (end 132.39534 89.4108) (width 0.25) (layer "F.Cu") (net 17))
 (segment (start 132.39642 86.41812) (end 132.39534 86.4192) (width 0.25) (layer "F.Cu") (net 17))
 (segment (start 130.88876 77.37348) (end 130.88876 86.41046) (width 0.25) (layer "F.Cu") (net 16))
 (segment (start 130.89642 86.41812) (end 130.89534 86.4192) (width 0.25) (layer "F.Cu") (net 16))
 (segment (start 130.89534 86.4192) (end 130.89534 89.4108) (width 0.25) (layer "F.Cu") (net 16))
 (segment (start 130.88876 86.41046) (end 130.89642 86.41812) (width 0.25) (layer "F.Cu") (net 16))
 (segment (start 129.39642 86.41812) (end 129.39534 86.4192) (width 0.25) (layer "F.Cu") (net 15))
 (segment (start 129.39534 86.4192) (end 129.39534 89.4108) (width 0.25) (layer "F.Cu") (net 15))
 (segment (start 129.38876 84.09546) (end 129.39642 84.10312) (width 0.25) (layer "F.Cu") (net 15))
 (segment (start 129.38876 77.37348) (end 129.38876 84.09546) (width 0.25) (layer "F.Cu") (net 15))
 (segment (start 129.39642 84.10312) (end 129.39642 86.41812) (width 0.25) (layer "F.Cu") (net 15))
 (segment (start 127.88876 89.40422) (end 127.89534 89.4108) (width 0.25) (layer "F.Cu") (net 14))
 (segment (start 127.88876 77.37348) (end 127.88876 89.40422) (width 0.25) (layer "F.Cu") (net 14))
 (segment (start 126.39534 86.41704) (end 126.39534 89.4108) (width 0.25) (layer "F.Cu") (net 13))
 (segment (start 126.38876 86.41046) (end 126.39534 86.41704) (width 0.25) (layer "F.Cu") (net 13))
 (segment (start 126.38876 86.41046) (end 126.39642 86.41812) (width 0.25) (layer "F.Cu") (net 13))
 (segment (start 126.38876 77.37348) (end 126.38876 86.41046) (width 0.25) (layer "F.Cu") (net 13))
 (segment (start 124.88876 77.37348) (end 124.88876 89.40422) (width 0.25) (layer "F.Cu") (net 12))
 (segment (start 124.88876 89.40422) (end 124.89534 89.4108) (width 0.25) (layer "F.Cu") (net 12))
 (segment (start 123.38876 77.37348) (end 123.38876 86.41046) (width 0.25) (layer "F.Cu") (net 11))
 (segment (start 123.39642 86.41812) (end 123.39534 86.4192) (width 0.25) (layer "F.Cu") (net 11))
 (segment (start 123.38876 86.41046) (end 123.39642 86.41812) (width 0.25) (layer "F.Cu") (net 11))
 (segment (start 123.39534 86.4192) (end 123.39534 89.4108) (width 0.25) (layer "F.Cu") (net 11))
 (segment (start 121.88876 77.37348) (end 121.88876 86.41046) (width 0.25) (layer "F.Cu") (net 10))
 (segment (start 121.89534 86.4192) (end 121.89534 89.4108) (width 0.25) (layer "F.Cu") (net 10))
 (segment (start 121.88876 86.41046) (end 121.89642 86.41812) (width 0.25) (layer "F.Cu") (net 10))
 (segment (start 121.89642 86.41812) (end 121.89534 86.4192) (width 0.25) (layer "F.Cu") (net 10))
 (segment (start 120.38876 77.37348) (end 120.38876 86.41046) (width 0.25) (layer "F.Cu") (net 9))
 (segment (start 120.39534 86.4192) (end 120.39534 89.4108) (width 0.25) (layer "F.Cu") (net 9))
 (segment (start 120.38876 86.41046) (end 120.39642 86.41812) (width 0.25) (layer "F.Cu") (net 9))
 (segment (start 120.39642 86.41812) (end 120.39534 86.4192) (width 0.25) (layer "F.Cu") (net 9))
 (segment (start 118.88876 86.19896) (end 118.89534 86.20554) (width 0.25) (layer "F.Cu") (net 8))
 (segment (start 118.88876 77.37348) (end 118.88876 86.19896) (width 0.25) (layer "F.Cu") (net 8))
 (segment (start 118.88876 86.19896) (end 118.88876 86.41046) (width 0.25) (layer "F.Cu") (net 8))
 (segment (start 118.88876 86.41046) (end 118.89642 86.41812) (width 0.25) (layer "F.Cu") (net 8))
 (segment (start 118.89534 86.20554) (end 118.89534 89.4108) (width 0.25) (layer "F.Cu") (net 8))
 (segment (start 117.38876 77.37348) (end 117.38876 89.40422) (width 0.25) (layer "F.Cu") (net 7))
 (segment (start 117.38876 89.40422) (end 117.39534 89.4108) (width 0.25) (layer "F.Cu") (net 7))
 (segment (start 115.89642 86.41812) (end 115.89534 86.4192) (width 0.25) (layer "F.Cu") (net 6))
 (segment (start 115.89534 86.4192) (end 115.89534 89.4108) (width 0.25) (layer "F.Cu") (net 6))
 (segment (start 115.88876 77.37348) (end 115.88876 86.41046) (width 0.25) (layer "F.Cu") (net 6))
 (segment (start 115.88876 86.41046) (end 115.89642 86.41812) (width 0.25) (layer "F.Cu") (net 6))
 (segment (start 114.39534 86.4192) (end 114.39534 89.4108) (width 0.25) (layer "F.Cu") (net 5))
 (segment (start 114.39642 86.41812) (end 114.39534 86.4192) (width 0.25) (layer "F.Cu") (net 5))
 (segment (start 114.38876 86.41046) (end 114.39642 86.41812) (width 0.25) (layer "F.Cu") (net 5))
 (segment (start 114.38876 77.37348) (end 114.38876 86.41046) (width 0.25) (layer "F.Cu") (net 5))
 (segment (start 112.89534 89.4108) (end 112.89534 77.38006) (width 0.25) (layer "F.Cu") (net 4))
 (segment (start 112.89534 77.38006) (end 112.88876 77.37348) (width 0.25) (layer "F.Cu") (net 4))
 (segment (start 109.89534 86.4192) (end 109.89534 89.4108) (width 0.25) (layer "F.Cu") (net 2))
 (segment (start 109.88876 77.37348) (end 109.88876 86.41046) (width 0.25) (layer "F.Cu") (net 2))
 (segment (start 109.89642 86.41812) (end 109.89534 86.4192) (width 0.25) (layer "F.Cu") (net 2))
 (segment (start 109.88876 86.41046) (end 109.89642 86.41812) (width 0.25) (layer "F.Cu") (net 2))
 (segment (start 108.39046 77.37322) (end 106.8578 78.90588) (width 0.25) (layer "F.Cu") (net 1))
 (segment (start 106.8578 83.947) (end 108.39704 85.48624) (width 0.25) (layer "F.Cu") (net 1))
 (segment (start 106.8578 78.90588) (end 106.8578 83.947) (width 0.25) (layer "F.Cu") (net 1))
 (segment (start 108.39704 85.48624) (end 108.39704 89.41054) (width 0.25) (layer "F.Cu") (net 1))
 (segment (start 105.3592 80.24474) (end 103.90526 78.7908) (width 0.25) (layer "F.Cu") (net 33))
 (segment (start 103.90526 78.7908) (end 101.473 78.7908) (width 0.25) (layer "F.Cu") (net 33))
 (segment (start 105.3592 81.3054) (end 105.3592 80.24474) (width 0.25) (layer "F.Cu") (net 33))
 (segment (start 101.473 78.7908) (end 98.9838 81.28) (width 0.25) (layer "F.Cu") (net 33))
 (segment (start 102.8374 78.3408) (end 101.531 78.3408) (width 0.25) (layer "F.Cu") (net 34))
 (segment (start 101.531 78.3408) (end 98.9838 75.7936) (width 0.25) (layer "F.Cu") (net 34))
 (segment (start 105.3592 75.819) (end 102.8374 78.3408) (width 0.25) (layer "F.Cu") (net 34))
 (segment (start 102.4382 76.2) (end 102.0318 75.7936) (width 0.25) (layer "F.Cu") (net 35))
 (segment (start 102.4382 77.5462) (end 102.4382 76.2) (width 0.25) (layer "F.Cu") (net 35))
 (via (at 102.4382 77.5462) (size 0.8) (drill 0.4) (layers "F.Cu" "B.Cu") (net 35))
 (segment (start 106.9848 75.7334) (end 106.9848 76.9366) (width 0.25) (layer "B.Cu") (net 35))
 (segment (start 106.9848 76.9366) (end 106.3752 77.5462) (width 0.25) (layer "B.Cu") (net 35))
 (segment (start 108.4072 75.311) (end 107.4072 75.311) (width 0.25) (layer "B.Cu") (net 35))
 (segment (start 106.3752 77.5462) (end 102.4382 77.5462) (width 0.25) (layer "B.Cu") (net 35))
 (segment (start 107.4072 75.311) (end 106.9848 75.7334) (width 0.25) (layer "B.Cu") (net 35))
 (segment (start 103.2764 80.0354) (end 102.0318 81.28) (width 0.25) (layer "F.Cu") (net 36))
 (segment (start 103.2764 79.8576) (end 103.2764 80.0354) (width 0.25) (layer "F.Cu") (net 36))
 (via (at 103.2764 79.8576) (size 0.8) (drill 0.4) (layers "F.Cu" "B.Cu") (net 36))
 (segment (start 108.4072 81.3054) (end 106.9594 79.8576) (width 0.25) (layer "B.Cu") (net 36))
 (segment (start 106.9594 79.8576) (end 103.2764 79.8576) (width 0.25) (layer "B.Cu") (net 36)))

